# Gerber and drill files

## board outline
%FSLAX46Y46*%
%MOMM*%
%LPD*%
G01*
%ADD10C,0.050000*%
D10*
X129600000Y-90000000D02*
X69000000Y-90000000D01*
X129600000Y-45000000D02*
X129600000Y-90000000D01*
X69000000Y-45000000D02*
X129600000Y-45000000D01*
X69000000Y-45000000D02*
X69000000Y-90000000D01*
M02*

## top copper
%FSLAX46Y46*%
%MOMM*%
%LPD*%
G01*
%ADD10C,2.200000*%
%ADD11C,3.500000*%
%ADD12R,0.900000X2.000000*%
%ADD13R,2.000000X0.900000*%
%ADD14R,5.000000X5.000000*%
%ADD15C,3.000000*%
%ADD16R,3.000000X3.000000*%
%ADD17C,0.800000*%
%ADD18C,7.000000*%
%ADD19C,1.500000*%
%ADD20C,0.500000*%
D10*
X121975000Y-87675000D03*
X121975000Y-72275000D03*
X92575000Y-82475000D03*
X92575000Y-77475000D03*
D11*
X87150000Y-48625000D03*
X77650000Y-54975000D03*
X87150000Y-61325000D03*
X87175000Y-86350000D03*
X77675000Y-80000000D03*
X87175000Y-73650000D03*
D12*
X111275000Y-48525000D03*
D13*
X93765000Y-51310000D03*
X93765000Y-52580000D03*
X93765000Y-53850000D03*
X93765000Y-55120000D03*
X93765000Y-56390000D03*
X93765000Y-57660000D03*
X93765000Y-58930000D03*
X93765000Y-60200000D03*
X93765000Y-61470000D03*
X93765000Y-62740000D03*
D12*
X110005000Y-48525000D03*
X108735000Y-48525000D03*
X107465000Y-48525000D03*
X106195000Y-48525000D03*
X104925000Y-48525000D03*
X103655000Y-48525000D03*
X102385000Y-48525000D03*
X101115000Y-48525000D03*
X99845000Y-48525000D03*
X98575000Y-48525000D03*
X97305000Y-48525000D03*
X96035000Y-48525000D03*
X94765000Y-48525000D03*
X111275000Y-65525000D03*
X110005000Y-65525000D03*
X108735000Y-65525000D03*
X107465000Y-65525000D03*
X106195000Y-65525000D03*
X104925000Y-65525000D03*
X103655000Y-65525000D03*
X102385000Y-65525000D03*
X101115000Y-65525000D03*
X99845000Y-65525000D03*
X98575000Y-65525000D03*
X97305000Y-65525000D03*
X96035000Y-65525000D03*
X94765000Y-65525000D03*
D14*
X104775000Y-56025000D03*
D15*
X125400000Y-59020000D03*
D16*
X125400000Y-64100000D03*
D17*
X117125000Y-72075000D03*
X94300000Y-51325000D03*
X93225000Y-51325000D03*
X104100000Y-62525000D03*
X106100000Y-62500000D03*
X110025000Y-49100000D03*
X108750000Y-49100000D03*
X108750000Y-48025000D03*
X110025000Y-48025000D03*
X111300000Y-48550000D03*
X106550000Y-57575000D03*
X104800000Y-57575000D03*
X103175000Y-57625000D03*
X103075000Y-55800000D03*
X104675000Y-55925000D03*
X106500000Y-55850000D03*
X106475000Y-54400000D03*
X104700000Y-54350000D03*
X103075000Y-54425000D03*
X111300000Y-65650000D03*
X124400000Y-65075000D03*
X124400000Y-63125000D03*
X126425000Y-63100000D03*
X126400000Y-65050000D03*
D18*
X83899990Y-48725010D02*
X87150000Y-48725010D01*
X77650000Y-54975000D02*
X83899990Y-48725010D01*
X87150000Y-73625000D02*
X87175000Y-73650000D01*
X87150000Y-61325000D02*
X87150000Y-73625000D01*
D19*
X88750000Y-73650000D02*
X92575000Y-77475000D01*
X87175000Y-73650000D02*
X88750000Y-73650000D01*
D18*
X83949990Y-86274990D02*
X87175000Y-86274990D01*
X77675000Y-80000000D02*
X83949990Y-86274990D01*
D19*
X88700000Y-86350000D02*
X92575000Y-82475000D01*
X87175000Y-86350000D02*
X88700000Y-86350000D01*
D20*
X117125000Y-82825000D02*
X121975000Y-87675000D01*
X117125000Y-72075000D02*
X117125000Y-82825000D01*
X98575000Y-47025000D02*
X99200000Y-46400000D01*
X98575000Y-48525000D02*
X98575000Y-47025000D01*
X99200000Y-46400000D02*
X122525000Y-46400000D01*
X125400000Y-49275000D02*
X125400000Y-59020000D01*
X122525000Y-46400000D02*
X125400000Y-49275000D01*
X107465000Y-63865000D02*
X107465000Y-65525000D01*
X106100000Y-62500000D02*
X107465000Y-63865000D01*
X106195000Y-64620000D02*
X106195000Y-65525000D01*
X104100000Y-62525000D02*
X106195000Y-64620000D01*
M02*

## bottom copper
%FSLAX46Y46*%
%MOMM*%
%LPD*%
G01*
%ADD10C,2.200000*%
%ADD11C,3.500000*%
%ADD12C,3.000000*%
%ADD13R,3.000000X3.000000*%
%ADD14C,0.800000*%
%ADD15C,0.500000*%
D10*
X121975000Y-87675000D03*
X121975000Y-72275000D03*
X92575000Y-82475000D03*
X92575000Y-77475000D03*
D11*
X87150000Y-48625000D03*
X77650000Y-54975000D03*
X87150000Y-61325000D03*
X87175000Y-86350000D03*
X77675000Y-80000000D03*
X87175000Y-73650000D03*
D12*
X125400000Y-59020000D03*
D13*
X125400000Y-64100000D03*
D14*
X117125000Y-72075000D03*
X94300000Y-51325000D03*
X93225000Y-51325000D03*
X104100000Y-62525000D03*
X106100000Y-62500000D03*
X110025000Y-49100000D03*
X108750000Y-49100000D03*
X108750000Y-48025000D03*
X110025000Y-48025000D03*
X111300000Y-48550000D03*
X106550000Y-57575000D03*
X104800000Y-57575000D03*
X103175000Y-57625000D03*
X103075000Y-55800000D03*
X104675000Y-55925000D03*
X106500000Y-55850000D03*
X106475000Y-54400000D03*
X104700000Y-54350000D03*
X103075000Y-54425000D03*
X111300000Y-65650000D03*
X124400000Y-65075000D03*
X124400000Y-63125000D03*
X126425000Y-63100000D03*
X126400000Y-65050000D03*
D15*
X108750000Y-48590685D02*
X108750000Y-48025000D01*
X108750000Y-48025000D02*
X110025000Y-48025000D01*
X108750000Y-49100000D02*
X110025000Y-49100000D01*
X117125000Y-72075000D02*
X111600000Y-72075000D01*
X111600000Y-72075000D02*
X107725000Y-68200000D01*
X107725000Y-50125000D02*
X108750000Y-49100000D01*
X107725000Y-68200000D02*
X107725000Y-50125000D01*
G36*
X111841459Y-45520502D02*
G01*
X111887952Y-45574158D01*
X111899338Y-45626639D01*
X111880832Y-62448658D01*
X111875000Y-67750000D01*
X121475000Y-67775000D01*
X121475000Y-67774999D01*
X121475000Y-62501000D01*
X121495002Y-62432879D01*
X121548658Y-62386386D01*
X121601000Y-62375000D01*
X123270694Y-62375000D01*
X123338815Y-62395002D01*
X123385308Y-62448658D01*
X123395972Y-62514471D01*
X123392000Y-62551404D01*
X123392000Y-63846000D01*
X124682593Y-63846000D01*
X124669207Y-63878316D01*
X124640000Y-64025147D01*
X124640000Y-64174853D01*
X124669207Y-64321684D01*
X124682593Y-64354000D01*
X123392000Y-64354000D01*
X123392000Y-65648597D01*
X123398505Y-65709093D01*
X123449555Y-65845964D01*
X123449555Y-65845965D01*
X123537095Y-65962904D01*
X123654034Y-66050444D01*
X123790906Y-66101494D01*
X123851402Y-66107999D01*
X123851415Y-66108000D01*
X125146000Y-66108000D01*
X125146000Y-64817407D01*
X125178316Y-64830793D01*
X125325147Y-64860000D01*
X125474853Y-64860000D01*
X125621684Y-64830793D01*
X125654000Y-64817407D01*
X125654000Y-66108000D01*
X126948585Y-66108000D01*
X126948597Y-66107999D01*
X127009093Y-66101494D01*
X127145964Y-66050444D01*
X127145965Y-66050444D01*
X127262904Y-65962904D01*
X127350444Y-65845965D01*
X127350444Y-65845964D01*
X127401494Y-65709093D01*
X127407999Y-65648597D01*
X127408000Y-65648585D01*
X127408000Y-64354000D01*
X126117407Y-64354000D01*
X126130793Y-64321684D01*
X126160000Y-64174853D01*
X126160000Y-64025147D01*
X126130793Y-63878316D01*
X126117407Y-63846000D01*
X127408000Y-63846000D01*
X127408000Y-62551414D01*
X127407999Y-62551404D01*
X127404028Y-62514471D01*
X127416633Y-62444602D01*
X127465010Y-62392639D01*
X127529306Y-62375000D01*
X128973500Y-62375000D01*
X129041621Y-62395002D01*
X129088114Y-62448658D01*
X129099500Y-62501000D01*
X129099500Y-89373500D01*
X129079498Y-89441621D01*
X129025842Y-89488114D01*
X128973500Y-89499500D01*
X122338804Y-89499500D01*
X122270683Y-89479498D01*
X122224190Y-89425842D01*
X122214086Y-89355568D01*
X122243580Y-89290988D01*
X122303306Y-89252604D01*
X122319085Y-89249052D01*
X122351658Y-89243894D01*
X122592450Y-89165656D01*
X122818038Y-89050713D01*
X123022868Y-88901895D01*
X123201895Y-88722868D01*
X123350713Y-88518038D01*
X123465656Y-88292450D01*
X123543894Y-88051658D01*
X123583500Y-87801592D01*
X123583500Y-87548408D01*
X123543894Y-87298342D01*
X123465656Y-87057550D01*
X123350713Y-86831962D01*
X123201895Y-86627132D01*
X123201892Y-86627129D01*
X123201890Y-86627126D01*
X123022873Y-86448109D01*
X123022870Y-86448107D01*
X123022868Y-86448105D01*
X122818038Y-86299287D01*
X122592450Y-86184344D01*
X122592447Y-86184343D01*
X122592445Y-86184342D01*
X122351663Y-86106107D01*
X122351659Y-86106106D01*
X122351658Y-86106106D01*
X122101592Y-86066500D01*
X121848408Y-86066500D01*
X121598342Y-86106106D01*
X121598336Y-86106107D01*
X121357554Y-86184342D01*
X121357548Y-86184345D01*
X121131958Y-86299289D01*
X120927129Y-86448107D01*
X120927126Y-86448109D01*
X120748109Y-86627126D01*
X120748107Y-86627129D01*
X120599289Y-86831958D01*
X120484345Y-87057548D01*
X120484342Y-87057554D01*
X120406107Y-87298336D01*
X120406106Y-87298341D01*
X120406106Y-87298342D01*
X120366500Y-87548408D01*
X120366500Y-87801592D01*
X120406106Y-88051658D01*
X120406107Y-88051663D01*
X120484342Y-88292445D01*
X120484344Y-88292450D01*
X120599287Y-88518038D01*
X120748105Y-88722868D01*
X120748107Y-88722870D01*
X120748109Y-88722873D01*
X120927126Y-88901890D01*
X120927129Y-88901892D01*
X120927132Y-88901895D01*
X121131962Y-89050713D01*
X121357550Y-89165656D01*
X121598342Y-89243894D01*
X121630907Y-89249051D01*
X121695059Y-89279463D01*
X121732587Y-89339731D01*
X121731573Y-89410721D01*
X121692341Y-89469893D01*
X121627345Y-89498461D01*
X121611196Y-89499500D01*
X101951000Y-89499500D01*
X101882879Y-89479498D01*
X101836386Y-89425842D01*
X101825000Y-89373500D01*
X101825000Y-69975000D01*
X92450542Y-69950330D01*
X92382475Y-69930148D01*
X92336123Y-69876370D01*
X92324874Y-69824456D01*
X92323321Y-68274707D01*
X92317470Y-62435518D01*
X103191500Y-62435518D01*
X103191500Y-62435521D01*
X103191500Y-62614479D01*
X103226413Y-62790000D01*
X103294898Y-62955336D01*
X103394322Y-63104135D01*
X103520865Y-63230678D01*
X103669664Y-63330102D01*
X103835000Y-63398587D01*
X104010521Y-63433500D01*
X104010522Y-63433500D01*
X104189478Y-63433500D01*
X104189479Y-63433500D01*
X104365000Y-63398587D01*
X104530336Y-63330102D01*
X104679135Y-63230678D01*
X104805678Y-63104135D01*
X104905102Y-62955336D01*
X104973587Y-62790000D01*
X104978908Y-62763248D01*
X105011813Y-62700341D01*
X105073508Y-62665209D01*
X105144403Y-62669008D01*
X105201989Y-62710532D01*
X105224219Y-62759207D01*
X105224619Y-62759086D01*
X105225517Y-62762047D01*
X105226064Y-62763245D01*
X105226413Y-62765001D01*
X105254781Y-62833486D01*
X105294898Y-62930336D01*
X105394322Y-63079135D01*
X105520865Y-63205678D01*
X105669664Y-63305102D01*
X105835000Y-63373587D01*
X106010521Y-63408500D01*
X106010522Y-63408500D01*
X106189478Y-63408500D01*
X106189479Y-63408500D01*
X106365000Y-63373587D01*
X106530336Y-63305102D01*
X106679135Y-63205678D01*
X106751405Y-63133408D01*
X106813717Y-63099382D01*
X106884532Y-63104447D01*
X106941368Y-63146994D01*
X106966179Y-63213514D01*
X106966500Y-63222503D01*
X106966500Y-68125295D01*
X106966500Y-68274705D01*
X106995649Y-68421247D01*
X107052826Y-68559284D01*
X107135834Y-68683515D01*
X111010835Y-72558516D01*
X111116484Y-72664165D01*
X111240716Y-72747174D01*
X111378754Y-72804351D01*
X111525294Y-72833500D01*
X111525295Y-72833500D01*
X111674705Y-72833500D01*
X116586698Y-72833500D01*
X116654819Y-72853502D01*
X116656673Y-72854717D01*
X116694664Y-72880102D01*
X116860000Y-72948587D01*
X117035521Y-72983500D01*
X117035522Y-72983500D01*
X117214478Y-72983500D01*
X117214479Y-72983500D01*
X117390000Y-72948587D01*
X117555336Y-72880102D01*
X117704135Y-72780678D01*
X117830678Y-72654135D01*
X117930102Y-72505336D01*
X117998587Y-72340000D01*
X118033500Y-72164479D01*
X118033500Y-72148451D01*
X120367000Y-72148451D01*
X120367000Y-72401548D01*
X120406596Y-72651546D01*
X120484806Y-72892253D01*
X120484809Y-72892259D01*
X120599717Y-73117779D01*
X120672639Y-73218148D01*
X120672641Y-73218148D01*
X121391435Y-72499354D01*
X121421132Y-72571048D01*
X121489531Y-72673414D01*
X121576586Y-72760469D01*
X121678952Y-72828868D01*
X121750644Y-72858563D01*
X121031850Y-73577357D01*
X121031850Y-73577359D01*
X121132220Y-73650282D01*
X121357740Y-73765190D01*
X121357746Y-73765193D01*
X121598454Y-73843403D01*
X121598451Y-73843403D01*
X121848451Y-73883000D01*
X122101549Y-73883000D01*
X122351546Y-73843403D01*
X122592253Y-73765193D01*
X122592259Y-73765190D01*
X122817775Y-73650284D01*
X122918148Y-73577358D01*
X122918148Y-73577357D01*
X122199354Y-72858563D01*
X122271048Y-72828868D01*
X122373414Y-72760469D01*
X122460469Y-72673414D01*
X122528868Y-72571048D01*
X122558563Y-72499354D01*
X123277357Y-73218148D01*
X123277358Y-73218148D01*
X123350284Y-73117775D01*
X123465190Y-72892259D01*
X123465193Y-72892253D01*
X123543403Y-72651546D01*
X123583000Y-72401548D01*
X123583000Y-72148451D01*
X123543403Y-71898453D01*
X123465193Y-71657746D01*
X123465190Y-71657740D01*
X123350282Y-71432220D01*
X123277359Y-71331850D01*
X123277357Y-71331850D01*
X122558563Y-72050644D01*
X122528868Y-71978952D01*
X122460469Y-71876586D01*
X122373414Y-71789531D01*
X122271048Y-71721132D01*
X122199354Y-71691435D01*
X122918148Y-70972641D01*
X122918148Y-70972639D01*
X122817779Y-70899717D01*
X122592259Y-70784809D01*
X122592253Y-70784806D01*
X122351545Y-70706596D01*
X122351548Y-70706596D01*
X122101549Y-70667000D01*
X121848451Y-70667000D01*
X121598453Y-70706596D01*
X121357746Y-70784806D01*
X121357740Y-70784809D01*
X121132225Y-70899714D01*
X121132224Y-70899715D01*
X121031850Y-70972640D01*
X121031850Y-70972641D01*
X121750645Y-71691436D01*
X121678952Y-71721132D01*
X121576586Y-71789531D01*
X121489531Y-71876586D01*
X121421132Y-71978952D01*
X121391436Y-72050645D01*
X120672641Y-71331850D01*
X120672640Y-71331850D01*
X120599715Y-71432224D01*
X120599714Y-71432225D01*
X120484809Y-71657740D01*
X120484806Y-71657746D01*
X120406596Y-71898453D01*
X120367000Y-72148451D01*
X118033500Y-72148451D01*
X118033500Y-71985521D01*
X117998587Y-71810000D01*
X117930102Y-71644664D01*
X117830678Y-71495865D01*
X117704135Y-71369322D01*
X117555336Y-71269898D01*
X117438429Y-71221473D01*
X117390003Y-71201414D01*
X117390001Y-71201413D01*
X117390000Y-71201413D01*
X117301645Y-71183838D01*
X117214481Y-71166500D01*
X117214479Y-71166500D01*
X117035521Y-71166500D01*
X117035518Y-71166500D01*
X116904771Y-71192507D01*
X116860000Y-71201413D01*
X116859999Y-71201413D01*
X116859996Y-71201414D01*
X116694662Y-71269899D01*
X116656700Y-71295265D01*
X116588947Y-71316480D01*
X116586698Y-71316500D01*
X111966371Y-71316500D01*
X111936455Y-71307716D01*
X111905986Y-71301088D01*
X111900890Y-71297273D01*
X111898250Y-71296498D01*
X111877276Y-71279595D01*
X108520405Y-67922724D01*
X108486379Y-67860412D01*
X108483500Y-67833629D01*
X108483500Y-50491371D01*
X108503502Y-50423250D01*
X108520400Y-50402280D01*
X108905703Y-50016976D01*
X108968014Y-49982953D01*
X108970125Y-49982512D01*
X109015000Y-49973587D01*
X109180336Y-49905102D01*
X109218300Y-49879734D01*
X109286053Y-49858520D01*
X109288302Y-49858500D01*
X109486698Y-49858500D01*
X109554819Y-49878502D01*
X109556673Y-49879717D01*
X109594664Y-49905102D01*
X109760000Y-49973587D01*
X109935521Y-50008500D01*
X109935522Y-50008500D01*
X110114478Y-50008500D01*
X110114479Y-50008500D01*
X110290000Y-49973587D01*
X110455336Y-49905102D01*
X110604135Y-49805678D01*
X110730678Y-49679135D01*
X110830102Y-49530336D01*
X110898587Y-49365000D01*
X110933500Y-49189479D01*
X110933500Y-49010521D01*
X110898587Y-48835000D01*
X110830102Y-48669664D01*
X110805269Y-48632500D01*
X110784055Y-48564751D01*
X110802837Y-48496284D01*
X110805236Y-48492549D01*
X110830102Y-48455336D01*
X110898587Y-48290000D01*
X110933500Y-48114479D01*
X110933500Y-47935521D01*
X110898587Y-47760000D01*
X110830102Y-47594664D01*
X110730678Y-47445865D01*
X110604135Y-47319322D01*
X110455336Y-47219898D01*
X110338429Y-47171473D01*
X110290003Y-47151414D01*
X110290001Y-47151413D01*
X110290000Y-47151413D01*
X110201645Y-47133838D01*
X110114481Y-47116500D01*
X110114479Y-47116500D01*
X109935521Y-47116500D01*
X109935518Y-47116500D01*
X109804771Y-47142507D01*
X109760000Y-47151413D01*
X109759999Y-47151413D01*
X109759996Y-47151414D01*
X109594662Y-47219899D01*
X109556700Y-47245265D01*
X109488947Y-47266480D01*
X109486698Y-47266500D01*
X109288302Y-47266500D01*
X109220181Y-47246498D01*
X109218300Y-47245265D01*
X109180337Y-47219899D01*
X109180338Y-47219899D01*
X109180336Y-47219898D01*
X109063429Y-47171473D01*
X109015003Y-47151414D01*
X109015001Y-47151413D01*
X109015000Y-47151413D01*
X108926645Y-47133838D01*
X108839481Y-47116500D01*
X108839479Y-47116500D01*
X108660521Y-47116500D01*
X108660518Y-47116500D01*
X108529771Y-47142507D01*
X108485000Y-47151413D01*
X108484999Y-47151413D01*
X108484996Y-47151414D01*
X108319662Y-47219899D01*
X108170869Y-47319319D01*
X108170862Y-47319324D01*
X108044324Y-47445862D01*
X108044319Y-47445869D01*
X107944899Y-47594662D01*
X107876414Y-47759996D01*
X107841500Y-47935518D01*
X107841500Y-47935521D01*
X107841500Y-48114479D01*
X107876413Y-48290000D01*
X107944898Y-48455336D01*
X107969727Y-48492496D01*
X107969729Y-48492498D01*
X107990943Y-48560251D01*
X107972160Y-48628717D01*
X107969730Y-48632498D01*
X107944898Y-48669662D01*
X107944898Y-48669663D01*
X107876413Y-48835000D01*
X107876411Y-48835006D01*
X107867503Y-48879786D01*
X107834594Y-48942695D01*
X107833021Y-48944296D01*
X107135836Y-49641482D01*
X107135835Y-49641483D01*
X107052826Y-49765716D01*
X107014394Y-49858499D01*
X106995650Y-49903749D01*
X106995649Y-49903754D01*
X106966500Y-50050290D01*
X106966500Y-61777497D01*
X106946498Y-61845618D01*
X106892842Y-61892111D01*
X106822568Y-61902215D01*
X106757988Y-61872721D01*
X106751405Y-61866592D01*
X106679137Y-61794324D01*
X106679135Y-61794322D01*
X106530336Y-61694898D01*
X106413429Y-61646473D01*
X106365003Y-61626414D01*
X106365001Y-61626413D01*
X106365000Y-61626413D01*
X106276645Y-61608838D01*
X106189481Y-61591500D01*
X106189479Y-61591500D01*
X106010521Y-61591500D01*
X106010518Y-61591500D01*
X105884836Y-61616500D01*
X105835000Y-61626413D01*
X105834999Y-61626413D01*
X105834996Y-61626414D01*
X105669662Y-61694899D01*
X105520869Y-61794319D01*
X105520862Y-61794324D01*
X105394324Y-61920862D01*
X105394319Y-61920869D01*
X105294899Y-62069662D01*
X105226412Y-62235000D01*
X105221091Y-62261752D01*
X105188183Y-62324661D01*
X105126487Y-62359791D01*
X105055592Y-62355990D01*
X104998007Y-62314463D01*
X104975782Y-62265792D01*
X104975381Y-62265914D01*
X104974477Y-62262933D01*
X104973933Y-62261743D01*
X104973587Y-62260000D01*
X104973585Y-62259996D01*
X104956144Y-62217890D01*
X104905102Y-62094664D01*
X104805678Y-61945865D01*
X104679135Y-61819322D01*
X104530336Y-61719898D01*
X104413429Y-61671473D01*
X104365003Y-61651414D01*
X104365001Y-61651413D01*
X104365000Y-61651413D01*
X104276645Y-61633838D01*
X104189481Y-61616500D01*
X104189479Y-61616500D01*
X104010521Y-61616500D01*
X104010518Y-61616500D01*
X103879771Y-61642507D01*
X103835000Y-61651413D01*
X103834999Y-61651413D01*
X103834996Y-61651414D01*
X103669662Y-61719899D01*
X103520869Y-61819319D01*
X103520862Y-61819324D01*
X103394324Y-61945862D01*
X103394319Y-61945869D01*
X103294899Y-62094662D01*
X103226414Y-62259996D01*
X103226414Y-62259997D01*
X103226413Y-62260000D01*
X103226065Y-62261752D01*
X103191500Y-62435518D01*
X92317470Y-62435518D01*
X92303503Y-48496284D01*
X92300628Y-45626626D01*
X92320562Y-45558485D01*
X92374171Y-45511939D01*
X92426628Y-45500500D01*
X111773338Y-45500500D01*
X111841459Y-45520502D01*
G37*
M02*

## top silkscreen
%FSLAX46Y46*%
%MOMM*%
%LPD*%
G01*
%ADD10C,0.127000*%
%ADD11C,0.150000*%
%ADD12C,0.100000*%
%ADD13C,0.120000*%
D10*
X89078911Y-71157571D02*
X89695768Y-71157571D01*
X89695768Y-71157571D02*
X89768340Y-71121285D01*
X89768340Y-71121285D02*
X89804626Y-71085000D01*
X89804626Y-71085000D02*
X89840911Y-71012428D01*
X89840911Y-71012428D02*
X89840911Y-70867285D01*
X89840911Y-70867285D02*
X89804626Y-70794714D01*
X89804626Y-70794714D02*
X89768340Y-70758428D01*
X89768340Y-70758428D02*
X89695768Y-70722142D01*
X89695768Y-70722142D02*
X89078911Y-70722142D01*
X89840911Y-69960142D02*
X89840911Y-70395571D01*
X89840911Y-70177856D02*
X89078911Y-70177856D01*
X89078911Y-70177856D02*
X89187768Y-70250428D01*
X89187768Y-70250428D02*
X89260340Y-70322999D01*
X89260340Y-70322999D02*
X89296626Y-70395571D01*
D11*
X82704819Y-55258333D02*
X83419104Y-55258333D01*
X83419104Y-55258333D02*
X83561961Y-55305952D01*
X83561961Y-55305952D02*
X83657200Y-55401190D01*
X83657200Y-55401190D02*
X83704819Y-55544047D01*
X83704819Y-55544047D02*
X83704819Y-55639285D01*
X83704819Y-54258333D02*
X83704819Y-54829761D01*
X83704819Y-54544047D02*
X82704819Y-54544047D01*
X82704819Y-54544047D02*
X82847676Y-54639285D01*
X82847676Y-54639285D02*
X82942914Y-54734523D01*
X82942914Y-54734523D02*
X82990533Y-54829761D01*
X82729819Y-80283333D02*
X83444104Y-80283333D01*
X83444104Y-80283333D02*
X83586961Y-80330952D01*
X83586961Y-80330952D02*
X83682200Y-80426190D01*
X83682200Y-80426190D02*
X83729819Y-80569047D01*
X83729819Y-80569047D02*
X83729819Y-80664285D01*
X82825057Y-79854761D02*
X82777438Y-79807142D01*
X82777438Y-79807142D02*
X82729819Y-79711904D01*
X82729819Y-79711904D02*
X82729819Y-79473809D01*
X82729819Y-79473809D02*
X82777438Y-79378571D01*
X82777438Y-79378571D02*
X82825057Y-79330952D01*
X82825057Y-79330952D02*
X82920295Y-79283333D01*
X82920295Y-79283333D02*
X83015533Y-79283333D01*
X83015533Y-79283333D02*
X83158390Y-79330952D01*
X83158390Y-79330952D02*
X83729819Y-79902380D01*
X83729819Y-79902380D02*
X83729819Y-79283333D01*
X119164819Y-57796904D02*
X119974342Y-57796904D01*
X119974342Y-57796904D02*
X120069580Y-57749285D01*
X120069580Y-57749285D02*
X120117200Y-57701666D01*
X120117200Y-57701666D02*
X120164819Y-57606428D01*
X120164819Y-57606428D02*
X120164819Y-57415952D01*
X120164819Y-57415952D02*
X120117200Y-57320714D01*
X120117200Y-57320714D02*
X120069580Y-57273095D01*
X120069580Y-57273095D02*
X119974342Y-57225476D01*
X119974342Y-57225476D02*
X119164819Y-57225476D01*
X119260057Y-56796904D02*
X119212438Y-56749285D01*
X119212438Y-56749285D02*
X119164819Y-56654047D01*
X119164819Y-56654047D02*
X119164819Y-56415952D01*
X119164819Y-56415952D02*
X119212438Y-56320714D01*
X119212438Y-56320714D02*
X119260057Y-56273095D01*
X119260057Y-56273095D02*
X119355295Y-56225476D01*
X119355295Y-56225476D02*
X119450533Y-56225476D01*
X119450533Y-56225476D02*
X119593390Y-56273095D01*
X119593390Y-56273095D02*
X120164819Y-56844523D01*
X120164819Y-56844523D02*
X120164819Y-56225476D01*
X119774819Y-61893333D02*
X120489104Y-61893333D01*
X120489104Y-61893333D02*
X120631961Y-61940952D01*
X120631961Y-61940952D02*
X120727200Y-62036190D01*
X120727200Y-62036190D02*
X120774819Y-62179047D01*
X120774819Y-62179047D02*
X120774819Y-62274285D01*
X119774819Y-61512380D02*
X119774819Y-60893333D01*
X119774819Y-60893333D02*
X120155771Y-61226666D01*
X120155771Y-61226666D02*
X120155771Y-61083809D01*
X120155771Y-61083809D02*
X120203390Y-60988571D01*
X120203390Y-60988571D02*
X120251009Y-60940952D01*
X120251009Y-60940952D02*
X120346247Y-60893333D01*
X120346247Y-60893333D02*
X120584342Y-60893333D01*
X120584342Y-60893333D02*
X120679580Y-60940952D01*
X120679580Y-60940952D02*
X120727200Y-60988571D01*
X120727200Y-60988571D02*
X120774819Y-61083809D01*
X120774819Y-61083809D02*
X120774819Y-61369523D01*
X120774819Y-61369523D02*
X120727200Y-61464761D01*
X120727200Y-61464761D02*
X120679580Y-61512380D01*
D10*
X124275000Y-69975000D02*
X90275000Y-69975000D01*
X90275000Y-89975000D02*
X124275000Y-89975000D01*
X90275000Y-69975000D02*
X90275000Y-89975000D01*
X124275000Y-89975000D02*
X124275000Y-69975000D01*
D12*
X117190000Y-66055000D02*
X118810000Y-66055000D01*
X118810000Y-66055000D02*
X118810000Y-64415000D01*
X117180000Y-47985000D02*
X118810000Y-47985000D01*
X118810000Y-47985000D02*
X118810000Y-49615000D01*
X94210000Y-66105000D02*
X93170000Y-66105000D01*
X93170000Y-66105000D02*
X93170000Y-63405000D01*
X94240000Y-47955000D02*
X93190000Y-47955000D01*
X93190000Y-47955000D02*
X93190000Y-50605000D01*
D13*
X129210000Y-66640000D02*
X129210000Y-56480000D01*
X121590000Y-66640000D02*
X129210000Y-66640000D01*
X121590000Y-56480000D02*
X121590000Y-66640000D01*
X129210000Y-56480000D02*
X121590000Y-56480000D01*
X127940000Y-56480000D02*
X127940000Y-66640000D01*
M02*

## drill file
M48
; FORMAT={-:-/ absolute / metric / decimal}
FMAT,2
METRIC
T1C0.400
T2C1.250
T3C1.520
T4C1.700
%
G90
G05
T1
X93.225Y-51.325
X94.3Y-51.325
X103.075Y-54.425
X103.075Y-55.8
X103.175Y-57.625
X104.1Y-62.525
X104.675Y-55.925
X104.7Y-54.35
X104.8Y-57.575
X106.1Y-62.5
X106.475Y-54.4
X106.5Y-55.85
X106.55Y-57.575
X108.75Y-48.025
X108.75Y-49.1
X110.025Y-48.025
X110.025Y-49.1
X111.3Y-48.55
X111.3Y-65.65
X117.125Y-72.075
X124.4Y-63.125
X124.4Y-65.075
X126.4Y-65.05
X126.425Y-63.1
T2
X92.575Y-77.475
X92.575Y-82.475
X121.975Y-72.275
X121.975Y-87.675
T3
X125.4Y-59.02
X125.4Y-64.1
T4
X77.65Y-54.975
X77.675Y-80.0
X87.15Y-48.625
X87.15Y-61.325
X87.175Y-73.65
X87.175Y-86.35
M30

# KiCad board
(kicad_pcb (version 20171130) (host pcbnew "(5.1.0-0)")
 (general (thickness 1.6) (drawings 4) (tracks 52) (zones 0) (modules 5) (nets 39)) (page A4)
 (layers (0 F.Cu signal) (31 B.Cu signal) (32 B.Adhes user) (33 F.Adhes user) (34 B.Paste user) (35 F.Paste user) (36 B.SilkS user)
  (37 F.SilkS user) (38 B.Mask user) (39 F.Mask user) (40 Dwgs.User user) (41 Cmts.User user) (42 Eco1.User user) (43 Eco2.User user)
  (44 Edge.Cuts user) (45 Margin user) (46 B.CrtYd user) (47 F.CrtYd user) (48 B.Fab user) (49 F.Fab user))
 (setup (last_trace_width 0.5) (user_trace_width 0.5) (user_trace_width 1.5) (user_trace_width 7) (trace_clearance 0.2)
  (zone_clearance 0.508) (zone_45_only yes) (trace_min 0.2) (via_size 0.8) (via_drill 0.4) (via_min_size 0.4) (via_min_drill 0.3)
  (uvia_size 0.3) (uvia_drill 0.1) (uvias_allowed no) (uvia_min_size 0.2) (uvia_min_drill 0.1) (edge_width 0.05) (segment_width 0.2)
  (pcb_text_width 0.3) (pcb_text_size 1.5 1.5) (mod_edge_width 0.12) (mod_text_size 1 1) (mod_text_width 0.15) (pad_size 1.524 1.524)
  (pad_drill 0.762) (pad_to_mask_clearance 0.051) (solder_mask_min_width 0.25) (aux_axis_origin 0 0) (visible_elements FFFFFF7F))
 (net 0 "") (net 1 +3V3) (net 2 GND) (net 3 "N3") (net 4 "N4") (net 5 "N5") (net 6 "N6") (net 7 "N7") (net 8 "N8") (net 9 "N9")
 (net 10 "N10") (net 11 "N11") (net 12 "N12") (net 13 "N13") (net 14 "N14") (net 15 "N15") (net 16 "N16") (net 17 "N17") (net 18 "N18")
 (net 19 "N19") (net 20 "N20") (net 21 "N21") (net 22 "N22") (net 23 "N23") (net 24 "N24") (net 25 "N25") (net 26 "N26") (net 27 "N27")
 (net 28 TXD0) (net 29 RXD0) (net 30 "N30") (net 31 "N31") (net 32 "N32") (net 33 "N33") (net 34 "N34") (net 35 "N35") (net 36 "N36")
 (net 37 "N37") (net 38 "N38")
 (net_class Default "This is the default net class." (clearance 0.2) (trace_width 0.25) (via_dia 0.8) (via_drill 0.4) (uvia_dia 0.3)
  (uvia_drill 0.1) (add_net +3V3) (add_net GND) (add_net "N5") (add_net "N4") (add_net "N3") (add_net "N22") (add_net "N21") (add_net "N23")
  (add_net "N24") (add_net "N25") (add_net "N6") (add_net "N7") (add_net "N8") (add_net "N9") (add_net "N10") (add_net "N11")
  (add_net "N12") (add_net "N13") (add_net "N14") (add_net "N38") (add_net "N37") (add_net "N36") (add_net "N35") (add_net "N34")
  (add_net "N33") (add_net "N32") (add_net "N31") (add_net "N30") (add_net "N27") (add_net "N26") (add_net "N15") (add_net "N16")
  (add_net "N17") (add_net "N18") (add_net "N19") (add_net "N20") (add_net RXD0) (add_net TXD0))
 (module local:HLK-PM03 (layer F.Cu) (at 107.275 79.975)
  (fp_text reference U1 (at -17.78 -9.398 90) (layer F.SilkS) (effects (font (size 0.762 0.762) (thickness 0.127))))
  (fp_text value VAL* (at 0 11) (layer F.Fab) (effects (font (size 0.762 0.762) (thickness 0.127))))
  (fp_line (start 17 -10) (end -17 -10) (layer F.SilkS) (width 0.127))
  (fp_line (start -17 10) (end 17 10) (layer F.SilkS) (width 0.127))
  (fp_line (start -17 -10) (end -17 10) (layer F.SilkS) (width 0.127))
  (fp_line (start 17 10) (end 17 -10) (layer F.SilkS) (width 0.127))
  (pad 4 thru_hole circle (at 14.7 7.7) (size 2.2 2.2) (drill 1.25) (layers *.Cu *.Mask) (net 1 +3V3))
  (pad 3 thru_hole circle (at 14.7 -7.7) (size 2.2 2.2) (drill 1.25) (layers *.Cu *.Mask) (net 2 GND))
  (pad 2 thru_hole circle (at -14.7 2.5) (size 2.2 2.2) (drill 1.25) (layers *.Cu *.Mask) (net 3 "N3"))
  (pad 1 thru_hole circle (at -14.7 -2.5) (size 2.2 2.2) (drill 1.25) (layers *.Cu *.Mask) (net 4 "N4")))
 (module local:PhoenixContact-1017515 (layer F.Cu) (at 87.15 54.975 90)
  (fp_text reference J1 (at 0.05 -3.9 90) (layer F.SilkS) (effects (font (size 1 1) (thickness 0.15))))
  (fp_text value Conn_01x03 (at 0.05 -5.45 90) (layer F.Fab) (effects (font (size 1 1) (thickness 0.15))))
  (pad 1 thru_hole circle (at 6.35 0 90) (size 3.5 3.5) (drill 1.7) (layers *.Cu *.Mask) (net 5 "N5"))
  (pad 2 thru_hole circle (at 0 -9.5 90) (size 3.5 3.5) (drill 1.7) (layers *.Cu *.Mask) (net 5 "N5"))
  (pad 3 thru_hole circle (at -6.35 0 90) (size 3.5 3.5) (drill 1.7) (layers *.Cu *.Mask) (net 4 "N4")))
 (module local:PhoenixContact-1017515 (layer F.Cu) (at 87.175 80 90)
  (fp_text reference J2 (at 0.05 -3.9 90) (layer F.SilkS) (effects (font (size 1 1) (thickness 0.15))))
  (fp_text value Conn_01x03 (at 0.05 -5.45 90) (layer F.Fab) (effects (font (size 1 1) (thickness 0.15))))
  (pad 3 thru_hole circle (at -6.35 0 90) (size 3.5 3.5) (drill 1.7) (layers *.Cu *.Mask) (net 3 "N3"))
  (pad 2 thru_hole circle (at 0 -9.5 90) (size 3.5 3.5) (drill 1.7) (layers *.Cu *.Mask) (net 3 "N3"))
  (pad 1 thru_hole circle (at 6.35 0 90) (size 3.5 3.5) (drill 1.7) (layers *.Cu *.Mask) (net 4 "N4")))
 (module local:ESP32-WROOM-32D (layer F.Cu) (at 103.02 57.025 270)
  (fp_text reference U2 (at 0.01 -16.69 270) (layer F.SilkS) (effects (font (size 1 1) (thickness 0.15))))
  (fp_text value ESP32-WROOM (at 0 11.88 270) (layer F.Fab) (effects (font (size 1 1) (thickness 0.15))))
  (fp_line (start 9.03 -14.17) (end 9.03 -15.79) (layer F.SilkS) (width 0.1))
  (fp_line (start 9.03 -15.79) (end 7.39 -15.79) (layer F.SilkS) (width 0.1))
  (fp_line (start -9.04 -14.16) (end -9.04 -15.79) (layer F.SilkS) (width 0.1))
  (fp_line (start -9.04 -15.79) (end -7.41 -15.79) (layer F.SilkS) (width 0.1))
  (fp_line (start 9.08 8.81) (end 9.08 9.85) (layer F.SilkS) (width 0.1))
  (fp_line (start 9.08 9.85) (end 6.38 9.85) (layer F.SilkS) (width 0.1))
  (fp_line (start -9.07 8.78) (end -9.07 9.83) (layer F.SilkS) (width 0.1))
  (fp_line (start -9.07 9.83) (end -6.42 9.83) (layer F.SilkS) (width 0.1))
  (pad 1 smd rect (at -8.5 -8.255 270) (size 2 0.9) (layers F.Cu F.Paste F.Mask) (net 2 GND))
  (pad 15 smd rect (at -5.715 9.255) (size 2 0.9) (layers F.Cu F.Paste F.Mask) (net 2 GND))
  (pad 16 smd rect (at -4.445 9.255) (size 2 0.9) (layers F.Cu F.Paste F.Mask) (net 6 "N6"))
  (pad 17 smd rect (at -3.175 9.255) (size 2 0.9) (layers F.Cu F.Paste F.Mask) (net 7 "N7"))
  (pad 18 smd rect (at -1.905 9.255) (size 2 0.9) (layers F.Cu F.Paste F.Mask) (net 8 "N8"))
  (pad 19 smd rect (at -0.635 9.255) (size 2 0.9) (layers F.Cu F.Paste F.Mask) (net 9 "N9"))
  (pad 20 smd rect (at 0.635 9.255) (size 2 0.9) (layers F.Cu F.Paste F.Mask) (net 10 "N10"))
  (pad 21 smd rect (at 1.905 9.255) (size 2 0.9) (layers F.Cu F.Paste F.Mask) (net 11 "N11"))
  (pad 22 smd rect (at 3.175 9.255) (size 2 0.9) (layers F.Cu F.Paste F.Mask) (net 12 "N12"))
  (pad 23 smd rect (at 4.445 9.255) (size 2 0.9) (layers F.Cu F.Paste F.Mask) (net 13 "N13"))
  (pad 24 smd rect (at 5.715 9.255) (size 2 0.9) (layers F.Cu F.Paste F.Mask) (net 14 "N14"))
  (pad 2 smd rect (at -8.5 -6.985 270) (size 2 0.9) (layers F.Cu F.Paste F.Mask) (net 1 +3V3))
  (pad 3 smd rect (at -8.5 -5.715 270) (size 2 0.9) (layers F.Cu F.Paste F.Mask) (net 1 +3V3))
  (pad 4 smd rect (at -8.5 -4.445 270) (size 2 0.9) (layers F.Cu F.Paste F.Mask) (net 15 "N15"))
  (pad 5 smd rect (at -8.5 -3.175 270) (size 2 0.9) (layers F.Cu F.Paste F.Mask) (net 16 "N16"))
  (pad 6 smd rect (at -8.5 -1.905 270) (size 2 0.9) (layers F.Cu F.Paste F.Mask) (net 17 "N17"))
  (pad 7 smd rect (at -8.5 -0.635 270) (size 2 0.9) (layers F.Cu F.Paste F.Mask) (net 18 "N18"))
  (pad 8 smd rect (at -8.5 0.635 270) (size 2 0.9) (layers F.Cu F.Paste F.Mask) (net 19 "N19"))
  (pad 9 smd rect (at -8.5 1.905 270) (size 2 0.9) (layers F.Cu F.Paste F.Mask) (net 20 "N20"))
  (pad 10 smd rect (at -8.5 3.175 270) (size 2 0.9) (layers F.Cu F.Paste F.Mask) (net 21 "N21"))
  (pad 11 smd rect (at -8.5 4.445 270) (size 2 0.9) (layers F.Cu F.Paste F.Mask) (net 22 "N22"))
  (pad 12 smd rect (at -8.5 5.715 270) (size 2 0.9) (layers F.Cu F.Paste F.Mask) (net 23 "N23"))
  (pad 13 smd rect (at -8.5 6.985 270) (size 2 0.9) (layers F.Cu F.Paste F.Mask) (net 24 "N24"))
  (pad 14 smd rect (at -8.5 8.255 270) (size 2 0.9) (layers F.Cu F.Paste F.Mask) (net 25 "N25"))
  (pad 38 smd rect (at 8.5 -8.255 270) (size 2 0.9) (layers F.Cu F.Paste F.Mask) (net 2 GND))
  (pad 37 smd rect (at 8.5 -6.985 270) (size 2 0.9) (layers F.Cu F.Paste F.Mask) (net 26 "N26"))
  (pad 36 smd rect (at 8.5 -5.715 270) (size 2 0.9) (layers F.Cu F.Paste F.Mask) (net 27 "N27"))
  (pad 35 smd rect (at 8.5 -4.445 270) (size 2 0.9) (layers F.Cu F.Paste F.Mask) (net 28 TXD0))
  (pad 34 smd rect (at 8.5 -3.175 270) (size 2 0.9) (layers F.Cu F.Paste F.Mask) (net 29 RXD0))
  (pad 33 smd rect (at 8.5 -1.905 270) (size 2 0.9) (layers F.Cu F.Paste F.Mask) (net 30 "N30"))
  (pad 32 smd rect (at 8.5 -0.635 270) (size 2 0.9) (layers F.Cu F.Paste F.Mask) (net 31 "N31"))
  (pad 31 smd rect (at 8.5 0.635 270) (size 2 0.9) (layers F.Cu F.Paste F.Mask) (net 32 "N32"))
  (pad 30 smd rect (at 8.5 1.905 270) (size 2 0.9) (layers F.Cu F.Paste F.Mask) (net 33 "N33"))
  (pad 29 smd rect (at 8.5 3.175 270) (size 2 0.9) (layers F.Cu F.Paste F.Mask) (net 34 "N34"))
  (pad 28 smd rect (at 8.5 4.445 270) (size 2 0.9) (layers F.Cu F.Paste F.Mask) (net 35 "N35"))
  (pad 27 smd rect (at 8.5 5.715 270) (size 2 0.9) (layers F.Cu F.Paste F.Mask) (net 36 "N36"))
  (pad 26 smd rect (at 8.5 6.985 270) (size 2 0.9) (layers F.Cu F.Paste F.Mask) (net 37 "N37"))
  (pad 25 smd rect (at 8.5 8.255 270) (size 2 0.9) (layers F.Cu F.Paste F.Mask) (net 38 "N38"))
  (pad 39 smd rect (at -1 -1.755 270) (size 5 5) (layers F.Cu F.Paste F.Mask) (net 2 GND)))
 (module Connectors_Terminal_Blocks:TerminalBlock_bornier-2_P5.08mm (layer F.Cu) (at 125.4 64.1 90)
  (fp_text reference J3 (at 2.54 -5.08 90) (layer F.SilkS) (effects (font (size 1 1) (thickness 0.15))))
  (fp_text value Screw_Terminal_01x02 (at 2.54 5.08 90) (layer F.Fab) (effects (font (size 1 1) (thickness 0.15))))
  (fp_line (start -2.54 3.81) (end 7.62 3.81) (layer F.SilkS) (width 0.12))
  (fp_line (start -2.54 -3.81) (end -2.54 3.81) (layer F.SilkS) (width 0.12))
  (fp_line (start 7.62 -3.81) (end -2.54 -3.81) (layer F.SilkS) (width 0.12))
  (fp_line (start 7.62 3.81) (end 7.62 -3.81) (layer F.SilkS) (width 0.12))
  (fp_line (start 7.62 2.54) (end -2.54 2.54) (layer F.SilkS) (width 0.12))
  (pad 2 thru_hole circle (at 5.08 0 90) (size 3 3) (drill 1.52) (layers *.Cu *.Mask) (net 22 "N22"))
  (pad 1 thru_hole rect (at 0 0 90) (size 3 3) (drill 1.52) (layers *.Cu *.Mask) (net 2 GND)))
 (gr_line (start 129.6 90) (end 69 90) (layer Edge.Cuts) (width 0.05))
 (gr_line (start 129.6 45) (end 129.6 90) (layer Edge.Cuts) (width 0.05))
 (gr_line (start 69 45) (end 129.6 45) (layer Edge.Cuts) (width 0.05))
 (gr_line (start 69 45) (end 69 90) (layer Edge.Cuts) (width 0.05))
 (via (at 117.125 72.075) (size 0.8) (drill 0.4) (layers F.Cu B.Cu) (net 1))
 (via (at 94.3 51.325) (size 0.8) (drill 0.4) (layers F.Cu B.Cu) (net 2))
 (via (at 93.225 51.325) (size 0.8) (drill 0.4) (layers F.Cu B.Cu) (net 2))
 (via (at 104.1 62.525) (size 0.8) (drill 0.4) (layers F.Cu B.Cu) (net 29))
 (via (at 106.1 62.5) (size 0.8) (drill 0.4) (layers F.Cu B.Cu) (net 28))
 (via (at 110.025 49.1) (size 0.8) (drill 0.4) (layers F.Cu B.Cu) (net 1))
 (via (at 108.75 49.1) (size 0.8) (drill 0.4) (layers F.Cu B.Cu) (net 1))
 (via (at 108.75 48.025) (size 0.8) (drill 0.4) (layers F.Cu B.Cu) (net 1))
 (via (at 110.025 48.025) (size 0.8) (drill 0.4) (layers F.Cu B.Cu) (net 1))
 (via (at 111.3 48.55) (size 0.8) (drill 0.4) (layers F.Cu B.Cu) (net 2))
 (via (at 106.55 57.575) (size 0.8) (drill 0.4) (layers F.Cu B.Cu) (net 2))
 (via (at 104.8 57.575) (size 0.8) (drill 0.4) (layers F.Cu B.Cu) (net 2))
 (via (at 103.175 57.625) (size 0.8) (drill 0.4) (layers F.Cu B.Cu) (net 2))
 (via (at 103.075 55.8) (size 0.8) (drill 0.4) (layers F.Cu B.Cu) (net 2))
 (via (at 104.675 55.925) (size 0.8) (drill 0.4) (layers F.Cu B.Cu) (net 2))
 (via (at 106.5 55.85) (size 0.8) (drill 0.4) (layers F.Cu B.Cu) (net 2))
 (via (at 106.475 54.4) (size 0.8) (drill 0.4) (layers F.Cu B.Cu) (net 2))
 (via (at 104.7 54.35) (size 0.8) (drill 0.4) (layers F.Cu B.Cu) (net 2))
 (via (at 103.075 54.425) (size 0.8) (drill 0.4) (layers F.Cu B.Cu) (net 2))
 (via (at 111.3 65.65) (size 0.8) (drill 0.4) (layers F.Cu B.Cu) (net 2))
 (via (at 124.4 65.075) (size 0.8) (drill 0.4) (layers F.Cu B.Cu) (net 2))
 (via (at 124.4 63.125) (size 0.8) (drill 0.4) (layers F.Cu B.Cu) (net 2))
 (via (at 126.425 63.1) (size 0.8) (drill 0.4) (layers F.Cu B.Cu) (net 2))
 (via (at 126.4 65.05) (size 0.8) (drill 0.4) (layers F.Cu B.Cu) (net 2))
 (segment (start 83.89999 48.72501) (end 87.15 48.72501) (width 7) (layer F.Cu) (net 5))
 (segment (start 77.65 54.975) (end 83.89999 48.72501) (width 7) (layer F.Cu) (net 5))
 (segment (start 87.15 73.625) (end 87.175 73.65) (width 7) (layer F.Cu) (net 4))
 (segment (start 87.15 61.325) (end 87.15 73.625) (width 7) (layer F.Cu) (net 4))
 (segment (start 88.75 73.65) (end 92.575 77.475) (width 1.5) (layer F.Cu) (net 4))
 (segment (start 87.175 73.65) (end 88.75 73.65) (width 1.5) (layer F.Cu) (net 4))
 (segment (start 83.94999 86.27499) (end 87.175 86.27499) (width 7) (layer F.Cu) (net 3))
 (segment (start 77.675 80) (end 83.94999 86.27499) (width 7) (layer F.Cu) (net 3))
 (segment (start 88.7 86.35) (end 92.575 82.475) (width 1.5) (layer F.Cu) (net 3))
 (segment (start 87.175 86.35) (end 88.7 86.35) (width 1.5) (layer F.Cu) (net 3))
 (segment (start 117.125 82.825) (end 121.975 87.675) (width 0.5) (layer F.Cu) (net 1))
 (segment (start 117.125 72.075) (end 117.125 82.825) (width 0.5) (layer F.Cu) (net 1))
 (segment (start 108.75 48.590685) (end 108.75 48.025) (width 0.5) (layer B.Cu) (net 1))
 (segment (start 108.75 48.025) (end 110.025 48.025) (width 0.5) (layer B.Cu) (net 1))
 (segment (start 108.75 49.1) (end 110.025 49.1) (width 0.5) (layer B.Cu) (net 1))
 (segment (start 117.125 72.075) (end 111.6 72.075) (width 0.5) (layer B.Cu) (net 1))
 (segment (start 111.6 72.075) (end 107.725 68.2) (width 0.5) (layer B.Cu) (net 1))
 (segment (start 107.725 50.125) (end 108.75 49.1) (width 0.5) (layer B.Cu) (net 1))
 (segment (start 107.725 68.2) (end 107.725 50.125) (width 0.5) (layer B.Cu) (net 1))
 (segment (start 98.575 47.025) (end 99.2 46.4) (width 0.5) (layer F.Cu) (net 22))
 (segment (start 98.575 48.525) (end 98.575 47.025) (width 0.5) (layer F.Cu) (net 22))
 (segment (start 99.2 46.4) (end 122.525 46.4) (width 0.5) (layer F.Cu) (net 22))
 (segment (start 125.4 49.275) (end 125.4 59.02) (width 0.5) (layer F.Cu) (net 22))
 (segment (start 122.525 46.4) (end 125.4 49.275) (width 0.5) (layer F.Cu) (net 22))
 (segment (start 107.465 63.865) (end 107.465 65.525) (width 0.5) (layer F.Cu) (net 28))
 (segment (start 106.1 62.5) (end 107.465 63.865) (width 0.5) (layer F.Cu) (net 28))
 (segment (start 106.195 64.62) (end 106.195 65.525) (width 0.5) (layer F.Cu) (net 29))
 (segment (start 104.1 62.525) (end 106.195 64.62) (width 0.5) (layer F.Cu) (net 29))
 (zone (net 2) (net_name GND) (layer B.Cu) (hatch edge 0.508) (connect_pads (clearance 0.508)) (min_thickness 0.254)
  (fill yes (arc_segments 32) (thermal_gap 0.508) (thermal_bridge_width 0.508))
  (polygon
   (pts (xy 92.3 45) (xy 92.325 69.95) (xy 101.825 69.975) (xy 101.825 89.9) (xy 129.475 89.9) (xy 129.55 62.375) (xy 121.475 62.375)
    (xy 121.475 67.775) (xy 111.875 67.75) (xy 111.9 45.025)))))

